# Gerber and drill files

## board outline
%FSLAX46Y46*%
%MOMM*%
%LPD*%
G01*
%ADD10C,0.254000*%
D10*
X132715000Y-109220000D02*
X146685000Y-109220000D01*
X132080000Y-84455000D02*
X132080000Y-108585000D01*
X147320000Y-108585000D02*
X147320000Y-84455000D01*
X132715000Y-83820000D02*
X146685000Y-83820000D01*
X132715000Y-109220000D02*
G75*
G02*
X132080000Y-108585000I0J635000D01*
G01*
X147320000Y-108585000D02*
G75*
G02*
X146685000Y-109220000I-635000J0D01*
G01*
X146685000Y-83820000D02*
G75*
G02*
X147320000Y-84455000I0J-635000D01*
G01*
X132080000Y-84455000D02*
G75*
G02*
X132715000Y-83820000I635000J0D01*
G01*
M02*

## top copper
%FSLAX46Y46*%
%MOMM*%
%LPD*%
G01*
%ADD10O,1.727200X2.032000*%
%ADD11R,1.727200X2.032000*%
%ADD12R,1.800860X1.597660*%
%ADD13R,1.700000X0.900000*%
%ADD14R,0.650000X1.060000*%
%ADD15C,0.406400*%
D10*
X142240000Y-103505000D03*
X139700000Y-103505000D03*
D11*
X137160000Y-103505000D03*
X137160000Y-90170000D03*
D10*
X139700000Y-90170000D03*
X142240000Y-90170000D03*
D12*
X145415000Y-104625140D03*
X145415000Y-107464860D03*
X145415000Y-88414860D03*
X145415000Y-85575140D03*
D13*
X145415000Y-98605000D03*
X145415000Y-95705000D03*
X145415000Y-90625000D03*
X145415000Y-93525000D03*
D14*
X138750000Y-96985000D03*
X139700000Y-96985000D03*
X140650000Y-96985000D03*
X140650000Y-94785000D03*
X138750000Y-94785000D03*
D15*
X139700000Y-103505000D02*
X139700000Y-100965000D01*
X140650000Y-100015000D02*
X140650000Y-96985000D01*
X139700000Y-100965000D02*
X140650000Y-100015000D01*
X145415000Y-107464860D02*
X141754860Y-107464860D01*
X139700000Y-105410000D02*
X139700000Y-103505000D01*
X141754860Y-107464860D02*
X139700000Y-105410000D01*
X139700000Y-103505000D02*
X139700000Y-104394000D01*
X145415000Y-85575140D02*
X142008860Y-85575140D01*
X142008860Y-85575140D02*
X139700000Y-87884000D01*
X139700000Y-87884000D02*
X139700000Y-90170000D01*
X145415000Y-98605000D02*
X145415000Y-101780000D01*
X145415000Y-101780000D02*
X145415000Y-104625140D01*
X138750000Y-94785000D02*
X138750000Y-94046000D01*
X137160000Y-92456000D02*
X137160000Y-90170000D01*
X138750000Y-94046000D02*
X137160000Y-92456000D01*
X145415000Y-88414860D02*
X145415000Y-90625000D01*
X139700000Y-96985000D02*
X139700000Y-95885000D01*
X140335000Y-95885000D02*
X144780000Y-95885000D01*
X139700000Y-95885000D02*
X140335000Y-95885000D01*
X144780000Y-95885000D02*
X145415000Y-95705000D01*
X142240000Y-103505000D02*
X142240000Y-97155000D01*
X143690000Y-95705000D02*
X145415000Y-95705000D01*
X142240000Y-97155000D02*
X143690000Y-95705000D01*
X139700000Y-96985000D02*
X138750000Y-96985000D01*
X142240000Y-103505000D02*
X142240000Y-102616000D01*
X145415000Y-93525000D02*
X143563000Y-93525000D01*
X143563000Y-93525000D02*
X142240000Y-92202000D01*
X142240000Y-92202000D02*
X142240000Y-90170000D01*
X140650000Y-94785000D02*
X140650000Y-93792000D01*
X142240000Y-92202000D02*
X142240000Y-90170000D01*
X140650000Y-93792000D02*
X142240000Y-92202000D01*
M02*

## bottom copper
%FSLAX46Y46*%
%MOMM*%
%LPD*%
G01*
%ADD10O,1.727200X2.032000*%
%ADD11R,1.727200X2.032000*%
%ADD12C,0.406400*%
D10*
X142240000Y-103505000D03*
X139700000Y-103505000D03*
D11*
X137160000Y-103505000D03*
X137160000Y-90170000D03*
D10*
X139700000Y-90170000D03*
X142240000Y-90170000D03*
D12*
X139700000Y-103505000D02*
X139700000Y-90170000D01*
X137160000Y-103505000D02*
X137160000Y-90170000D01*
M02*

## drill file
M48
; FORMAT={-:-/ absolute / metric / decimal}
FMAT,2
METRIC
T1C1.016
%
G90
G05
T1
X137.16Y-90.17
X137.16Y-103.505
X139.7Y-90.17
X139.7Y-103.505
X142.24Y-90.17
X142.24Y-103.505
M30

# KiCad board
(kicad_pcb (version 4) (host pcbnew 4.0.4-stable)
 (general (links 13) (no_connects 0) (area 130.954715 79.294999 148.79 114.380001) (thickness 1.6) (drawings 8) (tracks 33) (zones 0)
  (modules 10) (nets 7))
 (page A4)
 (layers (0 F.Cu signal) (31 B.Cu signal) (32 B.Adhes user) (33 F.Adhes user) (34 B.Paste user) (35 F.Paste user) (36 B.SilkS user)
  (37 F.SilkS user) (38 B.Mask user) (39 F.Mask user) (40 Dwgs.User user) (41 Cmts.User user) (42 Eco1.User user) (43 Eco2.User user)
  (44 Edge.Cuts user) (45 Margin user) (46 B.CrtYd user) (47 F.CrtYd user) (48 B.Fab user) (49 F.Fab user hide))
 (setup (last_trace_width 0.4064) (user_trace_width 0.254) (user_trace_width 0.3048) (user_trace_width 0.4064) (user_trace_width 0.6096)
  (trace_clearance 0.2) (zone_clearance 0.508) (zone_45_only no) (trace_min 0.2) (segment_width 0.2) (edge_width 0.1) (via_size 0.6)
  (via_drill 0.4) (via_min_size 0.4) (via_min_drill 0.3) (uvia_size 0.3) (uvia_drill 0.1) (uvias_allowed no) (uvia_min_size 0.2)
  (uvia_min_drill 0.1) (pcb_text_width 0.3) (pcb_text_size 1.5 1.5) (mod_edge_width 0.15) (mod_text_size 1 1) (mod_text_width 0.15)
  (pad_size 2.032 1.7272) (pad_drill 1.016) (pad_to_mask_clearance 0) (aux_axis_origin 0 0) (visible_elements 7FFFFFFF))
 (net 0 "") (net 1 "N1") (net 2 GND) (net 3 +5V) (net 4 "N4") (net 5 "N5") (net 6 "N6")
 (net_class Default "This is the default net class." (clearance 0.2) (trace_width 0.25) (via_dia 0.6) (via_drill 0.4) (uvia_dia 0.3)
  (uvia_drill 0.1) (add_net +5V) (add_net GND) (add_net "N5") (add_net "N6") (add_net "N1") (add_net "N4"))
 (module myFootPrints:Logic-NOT (layer F.Cu) (at 139.7 95.25 90)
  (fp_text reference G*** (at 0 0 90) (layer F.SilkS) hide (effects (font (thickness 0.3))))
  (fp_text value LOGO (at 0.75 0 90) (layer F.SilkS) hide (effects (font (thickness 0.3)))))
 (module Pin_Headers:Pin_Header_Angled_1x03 (layer F.Cu) (at 142.24 103.505 270)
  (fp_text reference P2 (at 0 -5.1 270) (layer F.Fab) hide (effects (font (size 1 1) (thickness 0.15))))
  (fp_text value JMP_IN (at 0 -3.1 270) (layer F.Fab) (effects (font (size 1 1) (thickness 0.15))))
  (pad 1 thru_hole oval (at 0 0 270) (size 2.032 1.7272) (drill 1.016) (layers *.Cu *.Mask F.SilkS) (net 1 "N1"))
  (pad 2 thru_hole oval (at 0 2.54 270) (size 2.032 1.7272) (drill 1.016) (layers *.Cu *.Mask F.SilkS) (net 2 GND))
  (pad 3 thru_hole rect (at 0 5.08 270) (size 2.032 1.7272) (drill 1.016) (layers *.Cu *.Mask F.SilkS) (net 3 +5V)))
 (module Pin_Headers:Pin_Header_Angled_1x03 (layer F.Cu) (at 137.16 90.17 90)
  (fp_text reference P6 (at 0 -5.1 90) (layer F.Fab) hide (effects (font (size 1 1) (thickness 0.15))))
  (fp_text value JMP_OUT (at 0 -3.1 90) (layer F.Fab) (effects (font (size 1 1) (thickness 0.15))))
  (pad 1 thru_hole rect (at 0 0 90) (size 2.032 1.7272) (drill 1.016) (layers *.Cu *.Mask F.SilkS) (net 3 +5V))
  (pad 2 thru_hole oval (at 0 2.54 90) (size 2.032 1.7272) (drill 1.016) (layers *.Cu *.Mask F.SilkS) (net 2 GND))
  (pad 3 thru_hole oval (at 0 5.08 90) (size 2.032 1.7272) (drill 1.016) (layers *.Cu *.Mask F.SilkS) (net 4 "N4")))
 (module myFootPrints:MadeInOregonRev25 (layer F.Cu) (at 139.7 99.695)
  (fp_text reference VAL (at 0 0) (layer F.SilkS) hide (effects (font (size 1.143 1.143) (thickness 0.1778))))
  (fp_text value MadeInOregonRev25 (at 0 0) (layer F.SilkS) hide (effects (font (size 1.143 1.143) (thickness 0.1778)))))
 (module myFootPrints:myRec (layer F.Cu) (at 139.7 96.52)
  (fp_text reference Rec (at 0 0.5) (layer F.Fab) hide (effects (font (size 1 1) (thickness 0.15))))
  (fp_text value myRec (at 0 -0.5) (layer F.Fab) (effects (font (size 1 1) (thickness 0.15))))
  (fp_line (start -6.985 12.7) (end 6.985 12.7) (layer Edge.Cuts) (width 0.254))
  (fp_line (start -7.62 -12.065) (end -7.62 12.065) (layer Edge.Cuts) (width 0.254))
  (fp_line (start 7.62 12.065) (end 7.62 -12.065) (layer Edge.Cuts) (width 0.254))
  (fp_line (start -6.985 -12.7) (end 6.985 -12.7) (layer Edge.Cuts) (width 0.254))
  (fp_arc (start -6.985 12.065) (end -6.985 12.7) (angle 90) (layer Edge.Cuts) (width 0.254))
  (fp_arc (start 6.985 12.065) (end 7.62 12.065) (angle 90) (layer Edge.Cuts) (width 0.254))
  (fp_arc (start 6.985 -12.065) (end 6.985 -12.7) (angle 90) (layer Edge.Cuts) (width 0.254))
  (fp_arc (start -6.985 -12.065) (end -7.62 -12.065) (angle 90) (layer Edge.Cuts) (width 0.254)))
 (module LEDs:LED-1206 (layer F.Cu) (at 145.415 106.045 90)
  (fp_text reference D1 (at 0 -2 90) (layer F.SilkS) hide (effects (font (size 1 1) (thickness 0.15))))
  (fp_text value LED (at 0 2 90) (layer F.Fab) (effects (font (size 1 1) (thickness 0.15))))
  (pad 2 smd rect (at 1.41986 0 270) (size 1.59766 1.80086) (layers F.Cu F.Paste F.Mask) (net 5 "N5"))
  (pad 1 smd rect (at -1.41986 0 270) (size 1.59766 1.80086) (layers F.Cu F.Paste F.Mask) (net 2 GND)))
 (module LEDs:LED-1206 (layer F.Cu) (at 145.415 86.995 270)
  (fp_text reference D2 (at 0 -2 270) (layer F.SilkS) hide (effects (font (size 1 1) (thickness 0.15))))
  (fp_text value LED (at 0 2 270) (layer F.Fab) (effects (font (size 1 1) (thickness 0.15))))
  (pad 2 smd rect (at 1.41986 0 90) (size 1.59766 1.80086) (layers F.Cu F.Paste F.Mask) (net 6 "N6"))
  (pad 1 smd rect (at -1.41986 0 90) (size 1.59766 1.80086) (layers F.Cu F.Paste F.Mask) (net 2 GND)))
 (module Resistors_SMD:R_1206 (layer F.Cu) (at 145.415 97.155 90)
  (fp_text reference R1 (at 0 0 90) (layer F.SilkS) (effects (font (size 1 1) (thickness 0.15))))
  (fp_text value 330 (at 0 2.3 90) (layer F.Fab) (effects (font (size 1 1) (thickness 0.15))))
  (pad 1 smd rect (at -1.45 0 90) (size 0.9 1.7) (layers F.Cu F.Paste F.Mask) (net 5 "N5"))
  (pad 2 smd rect (at 1.45 0 90) (size 0.9 1.7) (layers F.Cu F.Paste F.Mask) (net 1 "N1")))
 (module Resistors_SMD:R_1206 (layer F.Cu) (at 145.415 92.075 270)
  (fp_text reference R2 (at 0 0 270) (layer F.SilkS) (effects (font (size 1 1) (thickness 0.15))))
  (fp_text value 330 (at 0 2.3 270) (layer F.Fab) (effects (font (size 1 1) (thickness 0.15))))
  (pad 1 smd rect (at -1.45 0 270) (size 0.9 1.7) (layers F.Cu F.Paste F.Mask) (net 6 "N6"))
  (pad 2 smd rect (at 1.45 0 270) (size 0.9 1.7) (layers F.Cu F.Paste F.Mask) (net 4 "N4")))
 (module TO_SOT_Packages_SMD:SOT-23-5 (layer F.Cu) (at 139.7 95.885 90)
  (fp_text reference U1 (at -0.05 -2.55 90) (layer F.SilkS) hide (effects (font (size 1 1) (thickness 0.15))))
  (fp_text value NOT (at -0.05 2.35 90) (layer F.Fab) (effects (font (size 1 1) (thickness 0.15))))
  (pad 1 smd rect (at -1.1 -0.95 90) (size 1.06 0.65) (layers F.Cu F.Paste F.Mask) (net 1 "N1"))
  (pad 2 smd rect (at -1.1 0 90) (size 1.06 0.65) (layers F.Cu F.Paste F.Mask) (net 1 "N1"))
  (pad 3 smd rect (at -1.1 0.95 90) (size 1.06 0.65) (layers F.Cu F.Paste F.Mask) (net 2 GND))
  (pad 4 smd rect (at 1.1 0.95 90) (size 1.06 0.65) (layers F.Cu F.Paste F.Mask) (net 4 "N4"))
  (pad 5 smd rect (at 1.1 -0.95 90) (size 1.06 0.65) (layers F.Cu F.Paste F.Mask) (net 3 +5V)))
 (segment (start 139.7 103.505) (end 139.7 100.965) (width 0.4064) (layer F.Cu) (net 2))
 (segment (start 140.65 100.015) (end 140.65 96.985) (width 0.4064) (layer F.Cu) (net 2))
 (segment (start 139.7 100.965) (end 140.65 100.015) (width 0.4064) (layer F.Cu) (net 2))
 (segment (start 145.415 107.46486) (end 141.75486 107.46486) (width 0.4064) (layer F.Cu) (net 2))
 (segment (start 139.7 105.41) (end 139.7 103.505) (width 0.4064) (layer F.Cu) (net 2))
 (segment (start 141.75486 107.46486) (end 139.7 105.41) (width 0.4064) (layer F.Cu) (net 2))
 (segment (start 139.7 103.505) (end 139.7 90.17) (width 0.4064) (layer B.Cu) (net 2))
 (segment (start 139.7 103.505) (end 139.7 104.394) (width 0.4064) (layer F.Cu) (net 2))
 (segment (start 145.415 85.57514) (end 142.00886 85.57514) (width 0.4064) (layer F.Cu) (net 2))
 (segment (start 142.00886 85.57514) (end 139.7 87.884) (width 0.4064) (layer F.Cu) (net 2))
 (segment (start 139.7 87.884) (end 139.7 90.17) (width 0.4064) (layer F.Cu) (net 2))
 (segment (start 145.415 98.605) (end 145.415 101.78) (width 0.4064) (layer F.Cu) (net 5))
 (segment (start 145.415 101.78) (end 145.415 104.62514) (width 0.4064) (layer F.Cu) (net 5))
 (segment (start 137.16 103.505) (end 137.16 90.17) (width 0.4064) (layer B.Cu) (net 3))
 (segment (start 138.75 94.785) (end 138.75 94.046) (width 0.4064) (layer F.Cu) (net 3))
 (segment (start 137.16 92.456) (end 137.16 90.17) (width 0.4064) (layer F.Cu) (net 3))
 (segment (start 138.75 94.046) (end 137.16 92.456) (width 0.4064) (layer F.Cu) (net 3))
 (segment (start 145.415 88.41486) (end 145.415 90.625) (width 0.4064) (layer F.Cu) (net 6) (status 20))
 (segment (start 139.7 96.985) (end 139.7 95.885) (width 0.4064) (layer F.Cu) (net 1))
 (segment (start 140.335 95.885) (end 144.78 95.885) (width 0.4064) (layer F.Cu) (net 1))
 (segment (start 139.7 95.885) (end 140.335 95.885) (width 0.4064) (layer F.Cu) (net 1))
 (segment (start 144.78 95.885) (end 145.415 95.705) (width 0.4064) (layer F.Cu) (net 1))
 (segment (start 142.24 103.505) (end 142.24 97.155) (width 0.4064) (layer F.Cu) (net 1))
 (segment (start 143.69 95.705) (end 145.415 95.705) (width 0.4064) (layer F.Cu) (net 1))
 (segment (start 142.24 97.155) (end 143.69 95.705) (width 0.4064) (layer F.Cu) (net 1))
 (segment (start 139.7 96.985) (end 138.75 96.985) (width 0.4064) (layer F.Cu) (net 1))
 (segment (start 142.24 103.505) (end 142.24 102.616) (width 0.4064) (layer F.Cu) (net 1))
 (segment (start 145.415 93.525) (end 143.563 93.525) (width 0.4064) (layer F.Cu) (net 4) (status 400000))
 (segment (start 143.563 93.525) (end 142.24 92.202) (width 0.4064) (layer F.Cu) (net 4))
 (segment (start 142.24 92.202) (end 142.24 90.17) (width 0.4064) (layer F.Cu) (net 4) (status 800000))
 (segment (start 140.65 94.785) (end 140.65 93.792) (width 0.4064) (layer F.Cu) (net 4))
 (segment (start 142.24 92.202) (end 142.24 90.17) (width 0.4064) (layer F.Cu) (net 4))
 (segment (start 140.65 93.792) (end 142.24 92.202) (width 0.4064) (layer F.Cu) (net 4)))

